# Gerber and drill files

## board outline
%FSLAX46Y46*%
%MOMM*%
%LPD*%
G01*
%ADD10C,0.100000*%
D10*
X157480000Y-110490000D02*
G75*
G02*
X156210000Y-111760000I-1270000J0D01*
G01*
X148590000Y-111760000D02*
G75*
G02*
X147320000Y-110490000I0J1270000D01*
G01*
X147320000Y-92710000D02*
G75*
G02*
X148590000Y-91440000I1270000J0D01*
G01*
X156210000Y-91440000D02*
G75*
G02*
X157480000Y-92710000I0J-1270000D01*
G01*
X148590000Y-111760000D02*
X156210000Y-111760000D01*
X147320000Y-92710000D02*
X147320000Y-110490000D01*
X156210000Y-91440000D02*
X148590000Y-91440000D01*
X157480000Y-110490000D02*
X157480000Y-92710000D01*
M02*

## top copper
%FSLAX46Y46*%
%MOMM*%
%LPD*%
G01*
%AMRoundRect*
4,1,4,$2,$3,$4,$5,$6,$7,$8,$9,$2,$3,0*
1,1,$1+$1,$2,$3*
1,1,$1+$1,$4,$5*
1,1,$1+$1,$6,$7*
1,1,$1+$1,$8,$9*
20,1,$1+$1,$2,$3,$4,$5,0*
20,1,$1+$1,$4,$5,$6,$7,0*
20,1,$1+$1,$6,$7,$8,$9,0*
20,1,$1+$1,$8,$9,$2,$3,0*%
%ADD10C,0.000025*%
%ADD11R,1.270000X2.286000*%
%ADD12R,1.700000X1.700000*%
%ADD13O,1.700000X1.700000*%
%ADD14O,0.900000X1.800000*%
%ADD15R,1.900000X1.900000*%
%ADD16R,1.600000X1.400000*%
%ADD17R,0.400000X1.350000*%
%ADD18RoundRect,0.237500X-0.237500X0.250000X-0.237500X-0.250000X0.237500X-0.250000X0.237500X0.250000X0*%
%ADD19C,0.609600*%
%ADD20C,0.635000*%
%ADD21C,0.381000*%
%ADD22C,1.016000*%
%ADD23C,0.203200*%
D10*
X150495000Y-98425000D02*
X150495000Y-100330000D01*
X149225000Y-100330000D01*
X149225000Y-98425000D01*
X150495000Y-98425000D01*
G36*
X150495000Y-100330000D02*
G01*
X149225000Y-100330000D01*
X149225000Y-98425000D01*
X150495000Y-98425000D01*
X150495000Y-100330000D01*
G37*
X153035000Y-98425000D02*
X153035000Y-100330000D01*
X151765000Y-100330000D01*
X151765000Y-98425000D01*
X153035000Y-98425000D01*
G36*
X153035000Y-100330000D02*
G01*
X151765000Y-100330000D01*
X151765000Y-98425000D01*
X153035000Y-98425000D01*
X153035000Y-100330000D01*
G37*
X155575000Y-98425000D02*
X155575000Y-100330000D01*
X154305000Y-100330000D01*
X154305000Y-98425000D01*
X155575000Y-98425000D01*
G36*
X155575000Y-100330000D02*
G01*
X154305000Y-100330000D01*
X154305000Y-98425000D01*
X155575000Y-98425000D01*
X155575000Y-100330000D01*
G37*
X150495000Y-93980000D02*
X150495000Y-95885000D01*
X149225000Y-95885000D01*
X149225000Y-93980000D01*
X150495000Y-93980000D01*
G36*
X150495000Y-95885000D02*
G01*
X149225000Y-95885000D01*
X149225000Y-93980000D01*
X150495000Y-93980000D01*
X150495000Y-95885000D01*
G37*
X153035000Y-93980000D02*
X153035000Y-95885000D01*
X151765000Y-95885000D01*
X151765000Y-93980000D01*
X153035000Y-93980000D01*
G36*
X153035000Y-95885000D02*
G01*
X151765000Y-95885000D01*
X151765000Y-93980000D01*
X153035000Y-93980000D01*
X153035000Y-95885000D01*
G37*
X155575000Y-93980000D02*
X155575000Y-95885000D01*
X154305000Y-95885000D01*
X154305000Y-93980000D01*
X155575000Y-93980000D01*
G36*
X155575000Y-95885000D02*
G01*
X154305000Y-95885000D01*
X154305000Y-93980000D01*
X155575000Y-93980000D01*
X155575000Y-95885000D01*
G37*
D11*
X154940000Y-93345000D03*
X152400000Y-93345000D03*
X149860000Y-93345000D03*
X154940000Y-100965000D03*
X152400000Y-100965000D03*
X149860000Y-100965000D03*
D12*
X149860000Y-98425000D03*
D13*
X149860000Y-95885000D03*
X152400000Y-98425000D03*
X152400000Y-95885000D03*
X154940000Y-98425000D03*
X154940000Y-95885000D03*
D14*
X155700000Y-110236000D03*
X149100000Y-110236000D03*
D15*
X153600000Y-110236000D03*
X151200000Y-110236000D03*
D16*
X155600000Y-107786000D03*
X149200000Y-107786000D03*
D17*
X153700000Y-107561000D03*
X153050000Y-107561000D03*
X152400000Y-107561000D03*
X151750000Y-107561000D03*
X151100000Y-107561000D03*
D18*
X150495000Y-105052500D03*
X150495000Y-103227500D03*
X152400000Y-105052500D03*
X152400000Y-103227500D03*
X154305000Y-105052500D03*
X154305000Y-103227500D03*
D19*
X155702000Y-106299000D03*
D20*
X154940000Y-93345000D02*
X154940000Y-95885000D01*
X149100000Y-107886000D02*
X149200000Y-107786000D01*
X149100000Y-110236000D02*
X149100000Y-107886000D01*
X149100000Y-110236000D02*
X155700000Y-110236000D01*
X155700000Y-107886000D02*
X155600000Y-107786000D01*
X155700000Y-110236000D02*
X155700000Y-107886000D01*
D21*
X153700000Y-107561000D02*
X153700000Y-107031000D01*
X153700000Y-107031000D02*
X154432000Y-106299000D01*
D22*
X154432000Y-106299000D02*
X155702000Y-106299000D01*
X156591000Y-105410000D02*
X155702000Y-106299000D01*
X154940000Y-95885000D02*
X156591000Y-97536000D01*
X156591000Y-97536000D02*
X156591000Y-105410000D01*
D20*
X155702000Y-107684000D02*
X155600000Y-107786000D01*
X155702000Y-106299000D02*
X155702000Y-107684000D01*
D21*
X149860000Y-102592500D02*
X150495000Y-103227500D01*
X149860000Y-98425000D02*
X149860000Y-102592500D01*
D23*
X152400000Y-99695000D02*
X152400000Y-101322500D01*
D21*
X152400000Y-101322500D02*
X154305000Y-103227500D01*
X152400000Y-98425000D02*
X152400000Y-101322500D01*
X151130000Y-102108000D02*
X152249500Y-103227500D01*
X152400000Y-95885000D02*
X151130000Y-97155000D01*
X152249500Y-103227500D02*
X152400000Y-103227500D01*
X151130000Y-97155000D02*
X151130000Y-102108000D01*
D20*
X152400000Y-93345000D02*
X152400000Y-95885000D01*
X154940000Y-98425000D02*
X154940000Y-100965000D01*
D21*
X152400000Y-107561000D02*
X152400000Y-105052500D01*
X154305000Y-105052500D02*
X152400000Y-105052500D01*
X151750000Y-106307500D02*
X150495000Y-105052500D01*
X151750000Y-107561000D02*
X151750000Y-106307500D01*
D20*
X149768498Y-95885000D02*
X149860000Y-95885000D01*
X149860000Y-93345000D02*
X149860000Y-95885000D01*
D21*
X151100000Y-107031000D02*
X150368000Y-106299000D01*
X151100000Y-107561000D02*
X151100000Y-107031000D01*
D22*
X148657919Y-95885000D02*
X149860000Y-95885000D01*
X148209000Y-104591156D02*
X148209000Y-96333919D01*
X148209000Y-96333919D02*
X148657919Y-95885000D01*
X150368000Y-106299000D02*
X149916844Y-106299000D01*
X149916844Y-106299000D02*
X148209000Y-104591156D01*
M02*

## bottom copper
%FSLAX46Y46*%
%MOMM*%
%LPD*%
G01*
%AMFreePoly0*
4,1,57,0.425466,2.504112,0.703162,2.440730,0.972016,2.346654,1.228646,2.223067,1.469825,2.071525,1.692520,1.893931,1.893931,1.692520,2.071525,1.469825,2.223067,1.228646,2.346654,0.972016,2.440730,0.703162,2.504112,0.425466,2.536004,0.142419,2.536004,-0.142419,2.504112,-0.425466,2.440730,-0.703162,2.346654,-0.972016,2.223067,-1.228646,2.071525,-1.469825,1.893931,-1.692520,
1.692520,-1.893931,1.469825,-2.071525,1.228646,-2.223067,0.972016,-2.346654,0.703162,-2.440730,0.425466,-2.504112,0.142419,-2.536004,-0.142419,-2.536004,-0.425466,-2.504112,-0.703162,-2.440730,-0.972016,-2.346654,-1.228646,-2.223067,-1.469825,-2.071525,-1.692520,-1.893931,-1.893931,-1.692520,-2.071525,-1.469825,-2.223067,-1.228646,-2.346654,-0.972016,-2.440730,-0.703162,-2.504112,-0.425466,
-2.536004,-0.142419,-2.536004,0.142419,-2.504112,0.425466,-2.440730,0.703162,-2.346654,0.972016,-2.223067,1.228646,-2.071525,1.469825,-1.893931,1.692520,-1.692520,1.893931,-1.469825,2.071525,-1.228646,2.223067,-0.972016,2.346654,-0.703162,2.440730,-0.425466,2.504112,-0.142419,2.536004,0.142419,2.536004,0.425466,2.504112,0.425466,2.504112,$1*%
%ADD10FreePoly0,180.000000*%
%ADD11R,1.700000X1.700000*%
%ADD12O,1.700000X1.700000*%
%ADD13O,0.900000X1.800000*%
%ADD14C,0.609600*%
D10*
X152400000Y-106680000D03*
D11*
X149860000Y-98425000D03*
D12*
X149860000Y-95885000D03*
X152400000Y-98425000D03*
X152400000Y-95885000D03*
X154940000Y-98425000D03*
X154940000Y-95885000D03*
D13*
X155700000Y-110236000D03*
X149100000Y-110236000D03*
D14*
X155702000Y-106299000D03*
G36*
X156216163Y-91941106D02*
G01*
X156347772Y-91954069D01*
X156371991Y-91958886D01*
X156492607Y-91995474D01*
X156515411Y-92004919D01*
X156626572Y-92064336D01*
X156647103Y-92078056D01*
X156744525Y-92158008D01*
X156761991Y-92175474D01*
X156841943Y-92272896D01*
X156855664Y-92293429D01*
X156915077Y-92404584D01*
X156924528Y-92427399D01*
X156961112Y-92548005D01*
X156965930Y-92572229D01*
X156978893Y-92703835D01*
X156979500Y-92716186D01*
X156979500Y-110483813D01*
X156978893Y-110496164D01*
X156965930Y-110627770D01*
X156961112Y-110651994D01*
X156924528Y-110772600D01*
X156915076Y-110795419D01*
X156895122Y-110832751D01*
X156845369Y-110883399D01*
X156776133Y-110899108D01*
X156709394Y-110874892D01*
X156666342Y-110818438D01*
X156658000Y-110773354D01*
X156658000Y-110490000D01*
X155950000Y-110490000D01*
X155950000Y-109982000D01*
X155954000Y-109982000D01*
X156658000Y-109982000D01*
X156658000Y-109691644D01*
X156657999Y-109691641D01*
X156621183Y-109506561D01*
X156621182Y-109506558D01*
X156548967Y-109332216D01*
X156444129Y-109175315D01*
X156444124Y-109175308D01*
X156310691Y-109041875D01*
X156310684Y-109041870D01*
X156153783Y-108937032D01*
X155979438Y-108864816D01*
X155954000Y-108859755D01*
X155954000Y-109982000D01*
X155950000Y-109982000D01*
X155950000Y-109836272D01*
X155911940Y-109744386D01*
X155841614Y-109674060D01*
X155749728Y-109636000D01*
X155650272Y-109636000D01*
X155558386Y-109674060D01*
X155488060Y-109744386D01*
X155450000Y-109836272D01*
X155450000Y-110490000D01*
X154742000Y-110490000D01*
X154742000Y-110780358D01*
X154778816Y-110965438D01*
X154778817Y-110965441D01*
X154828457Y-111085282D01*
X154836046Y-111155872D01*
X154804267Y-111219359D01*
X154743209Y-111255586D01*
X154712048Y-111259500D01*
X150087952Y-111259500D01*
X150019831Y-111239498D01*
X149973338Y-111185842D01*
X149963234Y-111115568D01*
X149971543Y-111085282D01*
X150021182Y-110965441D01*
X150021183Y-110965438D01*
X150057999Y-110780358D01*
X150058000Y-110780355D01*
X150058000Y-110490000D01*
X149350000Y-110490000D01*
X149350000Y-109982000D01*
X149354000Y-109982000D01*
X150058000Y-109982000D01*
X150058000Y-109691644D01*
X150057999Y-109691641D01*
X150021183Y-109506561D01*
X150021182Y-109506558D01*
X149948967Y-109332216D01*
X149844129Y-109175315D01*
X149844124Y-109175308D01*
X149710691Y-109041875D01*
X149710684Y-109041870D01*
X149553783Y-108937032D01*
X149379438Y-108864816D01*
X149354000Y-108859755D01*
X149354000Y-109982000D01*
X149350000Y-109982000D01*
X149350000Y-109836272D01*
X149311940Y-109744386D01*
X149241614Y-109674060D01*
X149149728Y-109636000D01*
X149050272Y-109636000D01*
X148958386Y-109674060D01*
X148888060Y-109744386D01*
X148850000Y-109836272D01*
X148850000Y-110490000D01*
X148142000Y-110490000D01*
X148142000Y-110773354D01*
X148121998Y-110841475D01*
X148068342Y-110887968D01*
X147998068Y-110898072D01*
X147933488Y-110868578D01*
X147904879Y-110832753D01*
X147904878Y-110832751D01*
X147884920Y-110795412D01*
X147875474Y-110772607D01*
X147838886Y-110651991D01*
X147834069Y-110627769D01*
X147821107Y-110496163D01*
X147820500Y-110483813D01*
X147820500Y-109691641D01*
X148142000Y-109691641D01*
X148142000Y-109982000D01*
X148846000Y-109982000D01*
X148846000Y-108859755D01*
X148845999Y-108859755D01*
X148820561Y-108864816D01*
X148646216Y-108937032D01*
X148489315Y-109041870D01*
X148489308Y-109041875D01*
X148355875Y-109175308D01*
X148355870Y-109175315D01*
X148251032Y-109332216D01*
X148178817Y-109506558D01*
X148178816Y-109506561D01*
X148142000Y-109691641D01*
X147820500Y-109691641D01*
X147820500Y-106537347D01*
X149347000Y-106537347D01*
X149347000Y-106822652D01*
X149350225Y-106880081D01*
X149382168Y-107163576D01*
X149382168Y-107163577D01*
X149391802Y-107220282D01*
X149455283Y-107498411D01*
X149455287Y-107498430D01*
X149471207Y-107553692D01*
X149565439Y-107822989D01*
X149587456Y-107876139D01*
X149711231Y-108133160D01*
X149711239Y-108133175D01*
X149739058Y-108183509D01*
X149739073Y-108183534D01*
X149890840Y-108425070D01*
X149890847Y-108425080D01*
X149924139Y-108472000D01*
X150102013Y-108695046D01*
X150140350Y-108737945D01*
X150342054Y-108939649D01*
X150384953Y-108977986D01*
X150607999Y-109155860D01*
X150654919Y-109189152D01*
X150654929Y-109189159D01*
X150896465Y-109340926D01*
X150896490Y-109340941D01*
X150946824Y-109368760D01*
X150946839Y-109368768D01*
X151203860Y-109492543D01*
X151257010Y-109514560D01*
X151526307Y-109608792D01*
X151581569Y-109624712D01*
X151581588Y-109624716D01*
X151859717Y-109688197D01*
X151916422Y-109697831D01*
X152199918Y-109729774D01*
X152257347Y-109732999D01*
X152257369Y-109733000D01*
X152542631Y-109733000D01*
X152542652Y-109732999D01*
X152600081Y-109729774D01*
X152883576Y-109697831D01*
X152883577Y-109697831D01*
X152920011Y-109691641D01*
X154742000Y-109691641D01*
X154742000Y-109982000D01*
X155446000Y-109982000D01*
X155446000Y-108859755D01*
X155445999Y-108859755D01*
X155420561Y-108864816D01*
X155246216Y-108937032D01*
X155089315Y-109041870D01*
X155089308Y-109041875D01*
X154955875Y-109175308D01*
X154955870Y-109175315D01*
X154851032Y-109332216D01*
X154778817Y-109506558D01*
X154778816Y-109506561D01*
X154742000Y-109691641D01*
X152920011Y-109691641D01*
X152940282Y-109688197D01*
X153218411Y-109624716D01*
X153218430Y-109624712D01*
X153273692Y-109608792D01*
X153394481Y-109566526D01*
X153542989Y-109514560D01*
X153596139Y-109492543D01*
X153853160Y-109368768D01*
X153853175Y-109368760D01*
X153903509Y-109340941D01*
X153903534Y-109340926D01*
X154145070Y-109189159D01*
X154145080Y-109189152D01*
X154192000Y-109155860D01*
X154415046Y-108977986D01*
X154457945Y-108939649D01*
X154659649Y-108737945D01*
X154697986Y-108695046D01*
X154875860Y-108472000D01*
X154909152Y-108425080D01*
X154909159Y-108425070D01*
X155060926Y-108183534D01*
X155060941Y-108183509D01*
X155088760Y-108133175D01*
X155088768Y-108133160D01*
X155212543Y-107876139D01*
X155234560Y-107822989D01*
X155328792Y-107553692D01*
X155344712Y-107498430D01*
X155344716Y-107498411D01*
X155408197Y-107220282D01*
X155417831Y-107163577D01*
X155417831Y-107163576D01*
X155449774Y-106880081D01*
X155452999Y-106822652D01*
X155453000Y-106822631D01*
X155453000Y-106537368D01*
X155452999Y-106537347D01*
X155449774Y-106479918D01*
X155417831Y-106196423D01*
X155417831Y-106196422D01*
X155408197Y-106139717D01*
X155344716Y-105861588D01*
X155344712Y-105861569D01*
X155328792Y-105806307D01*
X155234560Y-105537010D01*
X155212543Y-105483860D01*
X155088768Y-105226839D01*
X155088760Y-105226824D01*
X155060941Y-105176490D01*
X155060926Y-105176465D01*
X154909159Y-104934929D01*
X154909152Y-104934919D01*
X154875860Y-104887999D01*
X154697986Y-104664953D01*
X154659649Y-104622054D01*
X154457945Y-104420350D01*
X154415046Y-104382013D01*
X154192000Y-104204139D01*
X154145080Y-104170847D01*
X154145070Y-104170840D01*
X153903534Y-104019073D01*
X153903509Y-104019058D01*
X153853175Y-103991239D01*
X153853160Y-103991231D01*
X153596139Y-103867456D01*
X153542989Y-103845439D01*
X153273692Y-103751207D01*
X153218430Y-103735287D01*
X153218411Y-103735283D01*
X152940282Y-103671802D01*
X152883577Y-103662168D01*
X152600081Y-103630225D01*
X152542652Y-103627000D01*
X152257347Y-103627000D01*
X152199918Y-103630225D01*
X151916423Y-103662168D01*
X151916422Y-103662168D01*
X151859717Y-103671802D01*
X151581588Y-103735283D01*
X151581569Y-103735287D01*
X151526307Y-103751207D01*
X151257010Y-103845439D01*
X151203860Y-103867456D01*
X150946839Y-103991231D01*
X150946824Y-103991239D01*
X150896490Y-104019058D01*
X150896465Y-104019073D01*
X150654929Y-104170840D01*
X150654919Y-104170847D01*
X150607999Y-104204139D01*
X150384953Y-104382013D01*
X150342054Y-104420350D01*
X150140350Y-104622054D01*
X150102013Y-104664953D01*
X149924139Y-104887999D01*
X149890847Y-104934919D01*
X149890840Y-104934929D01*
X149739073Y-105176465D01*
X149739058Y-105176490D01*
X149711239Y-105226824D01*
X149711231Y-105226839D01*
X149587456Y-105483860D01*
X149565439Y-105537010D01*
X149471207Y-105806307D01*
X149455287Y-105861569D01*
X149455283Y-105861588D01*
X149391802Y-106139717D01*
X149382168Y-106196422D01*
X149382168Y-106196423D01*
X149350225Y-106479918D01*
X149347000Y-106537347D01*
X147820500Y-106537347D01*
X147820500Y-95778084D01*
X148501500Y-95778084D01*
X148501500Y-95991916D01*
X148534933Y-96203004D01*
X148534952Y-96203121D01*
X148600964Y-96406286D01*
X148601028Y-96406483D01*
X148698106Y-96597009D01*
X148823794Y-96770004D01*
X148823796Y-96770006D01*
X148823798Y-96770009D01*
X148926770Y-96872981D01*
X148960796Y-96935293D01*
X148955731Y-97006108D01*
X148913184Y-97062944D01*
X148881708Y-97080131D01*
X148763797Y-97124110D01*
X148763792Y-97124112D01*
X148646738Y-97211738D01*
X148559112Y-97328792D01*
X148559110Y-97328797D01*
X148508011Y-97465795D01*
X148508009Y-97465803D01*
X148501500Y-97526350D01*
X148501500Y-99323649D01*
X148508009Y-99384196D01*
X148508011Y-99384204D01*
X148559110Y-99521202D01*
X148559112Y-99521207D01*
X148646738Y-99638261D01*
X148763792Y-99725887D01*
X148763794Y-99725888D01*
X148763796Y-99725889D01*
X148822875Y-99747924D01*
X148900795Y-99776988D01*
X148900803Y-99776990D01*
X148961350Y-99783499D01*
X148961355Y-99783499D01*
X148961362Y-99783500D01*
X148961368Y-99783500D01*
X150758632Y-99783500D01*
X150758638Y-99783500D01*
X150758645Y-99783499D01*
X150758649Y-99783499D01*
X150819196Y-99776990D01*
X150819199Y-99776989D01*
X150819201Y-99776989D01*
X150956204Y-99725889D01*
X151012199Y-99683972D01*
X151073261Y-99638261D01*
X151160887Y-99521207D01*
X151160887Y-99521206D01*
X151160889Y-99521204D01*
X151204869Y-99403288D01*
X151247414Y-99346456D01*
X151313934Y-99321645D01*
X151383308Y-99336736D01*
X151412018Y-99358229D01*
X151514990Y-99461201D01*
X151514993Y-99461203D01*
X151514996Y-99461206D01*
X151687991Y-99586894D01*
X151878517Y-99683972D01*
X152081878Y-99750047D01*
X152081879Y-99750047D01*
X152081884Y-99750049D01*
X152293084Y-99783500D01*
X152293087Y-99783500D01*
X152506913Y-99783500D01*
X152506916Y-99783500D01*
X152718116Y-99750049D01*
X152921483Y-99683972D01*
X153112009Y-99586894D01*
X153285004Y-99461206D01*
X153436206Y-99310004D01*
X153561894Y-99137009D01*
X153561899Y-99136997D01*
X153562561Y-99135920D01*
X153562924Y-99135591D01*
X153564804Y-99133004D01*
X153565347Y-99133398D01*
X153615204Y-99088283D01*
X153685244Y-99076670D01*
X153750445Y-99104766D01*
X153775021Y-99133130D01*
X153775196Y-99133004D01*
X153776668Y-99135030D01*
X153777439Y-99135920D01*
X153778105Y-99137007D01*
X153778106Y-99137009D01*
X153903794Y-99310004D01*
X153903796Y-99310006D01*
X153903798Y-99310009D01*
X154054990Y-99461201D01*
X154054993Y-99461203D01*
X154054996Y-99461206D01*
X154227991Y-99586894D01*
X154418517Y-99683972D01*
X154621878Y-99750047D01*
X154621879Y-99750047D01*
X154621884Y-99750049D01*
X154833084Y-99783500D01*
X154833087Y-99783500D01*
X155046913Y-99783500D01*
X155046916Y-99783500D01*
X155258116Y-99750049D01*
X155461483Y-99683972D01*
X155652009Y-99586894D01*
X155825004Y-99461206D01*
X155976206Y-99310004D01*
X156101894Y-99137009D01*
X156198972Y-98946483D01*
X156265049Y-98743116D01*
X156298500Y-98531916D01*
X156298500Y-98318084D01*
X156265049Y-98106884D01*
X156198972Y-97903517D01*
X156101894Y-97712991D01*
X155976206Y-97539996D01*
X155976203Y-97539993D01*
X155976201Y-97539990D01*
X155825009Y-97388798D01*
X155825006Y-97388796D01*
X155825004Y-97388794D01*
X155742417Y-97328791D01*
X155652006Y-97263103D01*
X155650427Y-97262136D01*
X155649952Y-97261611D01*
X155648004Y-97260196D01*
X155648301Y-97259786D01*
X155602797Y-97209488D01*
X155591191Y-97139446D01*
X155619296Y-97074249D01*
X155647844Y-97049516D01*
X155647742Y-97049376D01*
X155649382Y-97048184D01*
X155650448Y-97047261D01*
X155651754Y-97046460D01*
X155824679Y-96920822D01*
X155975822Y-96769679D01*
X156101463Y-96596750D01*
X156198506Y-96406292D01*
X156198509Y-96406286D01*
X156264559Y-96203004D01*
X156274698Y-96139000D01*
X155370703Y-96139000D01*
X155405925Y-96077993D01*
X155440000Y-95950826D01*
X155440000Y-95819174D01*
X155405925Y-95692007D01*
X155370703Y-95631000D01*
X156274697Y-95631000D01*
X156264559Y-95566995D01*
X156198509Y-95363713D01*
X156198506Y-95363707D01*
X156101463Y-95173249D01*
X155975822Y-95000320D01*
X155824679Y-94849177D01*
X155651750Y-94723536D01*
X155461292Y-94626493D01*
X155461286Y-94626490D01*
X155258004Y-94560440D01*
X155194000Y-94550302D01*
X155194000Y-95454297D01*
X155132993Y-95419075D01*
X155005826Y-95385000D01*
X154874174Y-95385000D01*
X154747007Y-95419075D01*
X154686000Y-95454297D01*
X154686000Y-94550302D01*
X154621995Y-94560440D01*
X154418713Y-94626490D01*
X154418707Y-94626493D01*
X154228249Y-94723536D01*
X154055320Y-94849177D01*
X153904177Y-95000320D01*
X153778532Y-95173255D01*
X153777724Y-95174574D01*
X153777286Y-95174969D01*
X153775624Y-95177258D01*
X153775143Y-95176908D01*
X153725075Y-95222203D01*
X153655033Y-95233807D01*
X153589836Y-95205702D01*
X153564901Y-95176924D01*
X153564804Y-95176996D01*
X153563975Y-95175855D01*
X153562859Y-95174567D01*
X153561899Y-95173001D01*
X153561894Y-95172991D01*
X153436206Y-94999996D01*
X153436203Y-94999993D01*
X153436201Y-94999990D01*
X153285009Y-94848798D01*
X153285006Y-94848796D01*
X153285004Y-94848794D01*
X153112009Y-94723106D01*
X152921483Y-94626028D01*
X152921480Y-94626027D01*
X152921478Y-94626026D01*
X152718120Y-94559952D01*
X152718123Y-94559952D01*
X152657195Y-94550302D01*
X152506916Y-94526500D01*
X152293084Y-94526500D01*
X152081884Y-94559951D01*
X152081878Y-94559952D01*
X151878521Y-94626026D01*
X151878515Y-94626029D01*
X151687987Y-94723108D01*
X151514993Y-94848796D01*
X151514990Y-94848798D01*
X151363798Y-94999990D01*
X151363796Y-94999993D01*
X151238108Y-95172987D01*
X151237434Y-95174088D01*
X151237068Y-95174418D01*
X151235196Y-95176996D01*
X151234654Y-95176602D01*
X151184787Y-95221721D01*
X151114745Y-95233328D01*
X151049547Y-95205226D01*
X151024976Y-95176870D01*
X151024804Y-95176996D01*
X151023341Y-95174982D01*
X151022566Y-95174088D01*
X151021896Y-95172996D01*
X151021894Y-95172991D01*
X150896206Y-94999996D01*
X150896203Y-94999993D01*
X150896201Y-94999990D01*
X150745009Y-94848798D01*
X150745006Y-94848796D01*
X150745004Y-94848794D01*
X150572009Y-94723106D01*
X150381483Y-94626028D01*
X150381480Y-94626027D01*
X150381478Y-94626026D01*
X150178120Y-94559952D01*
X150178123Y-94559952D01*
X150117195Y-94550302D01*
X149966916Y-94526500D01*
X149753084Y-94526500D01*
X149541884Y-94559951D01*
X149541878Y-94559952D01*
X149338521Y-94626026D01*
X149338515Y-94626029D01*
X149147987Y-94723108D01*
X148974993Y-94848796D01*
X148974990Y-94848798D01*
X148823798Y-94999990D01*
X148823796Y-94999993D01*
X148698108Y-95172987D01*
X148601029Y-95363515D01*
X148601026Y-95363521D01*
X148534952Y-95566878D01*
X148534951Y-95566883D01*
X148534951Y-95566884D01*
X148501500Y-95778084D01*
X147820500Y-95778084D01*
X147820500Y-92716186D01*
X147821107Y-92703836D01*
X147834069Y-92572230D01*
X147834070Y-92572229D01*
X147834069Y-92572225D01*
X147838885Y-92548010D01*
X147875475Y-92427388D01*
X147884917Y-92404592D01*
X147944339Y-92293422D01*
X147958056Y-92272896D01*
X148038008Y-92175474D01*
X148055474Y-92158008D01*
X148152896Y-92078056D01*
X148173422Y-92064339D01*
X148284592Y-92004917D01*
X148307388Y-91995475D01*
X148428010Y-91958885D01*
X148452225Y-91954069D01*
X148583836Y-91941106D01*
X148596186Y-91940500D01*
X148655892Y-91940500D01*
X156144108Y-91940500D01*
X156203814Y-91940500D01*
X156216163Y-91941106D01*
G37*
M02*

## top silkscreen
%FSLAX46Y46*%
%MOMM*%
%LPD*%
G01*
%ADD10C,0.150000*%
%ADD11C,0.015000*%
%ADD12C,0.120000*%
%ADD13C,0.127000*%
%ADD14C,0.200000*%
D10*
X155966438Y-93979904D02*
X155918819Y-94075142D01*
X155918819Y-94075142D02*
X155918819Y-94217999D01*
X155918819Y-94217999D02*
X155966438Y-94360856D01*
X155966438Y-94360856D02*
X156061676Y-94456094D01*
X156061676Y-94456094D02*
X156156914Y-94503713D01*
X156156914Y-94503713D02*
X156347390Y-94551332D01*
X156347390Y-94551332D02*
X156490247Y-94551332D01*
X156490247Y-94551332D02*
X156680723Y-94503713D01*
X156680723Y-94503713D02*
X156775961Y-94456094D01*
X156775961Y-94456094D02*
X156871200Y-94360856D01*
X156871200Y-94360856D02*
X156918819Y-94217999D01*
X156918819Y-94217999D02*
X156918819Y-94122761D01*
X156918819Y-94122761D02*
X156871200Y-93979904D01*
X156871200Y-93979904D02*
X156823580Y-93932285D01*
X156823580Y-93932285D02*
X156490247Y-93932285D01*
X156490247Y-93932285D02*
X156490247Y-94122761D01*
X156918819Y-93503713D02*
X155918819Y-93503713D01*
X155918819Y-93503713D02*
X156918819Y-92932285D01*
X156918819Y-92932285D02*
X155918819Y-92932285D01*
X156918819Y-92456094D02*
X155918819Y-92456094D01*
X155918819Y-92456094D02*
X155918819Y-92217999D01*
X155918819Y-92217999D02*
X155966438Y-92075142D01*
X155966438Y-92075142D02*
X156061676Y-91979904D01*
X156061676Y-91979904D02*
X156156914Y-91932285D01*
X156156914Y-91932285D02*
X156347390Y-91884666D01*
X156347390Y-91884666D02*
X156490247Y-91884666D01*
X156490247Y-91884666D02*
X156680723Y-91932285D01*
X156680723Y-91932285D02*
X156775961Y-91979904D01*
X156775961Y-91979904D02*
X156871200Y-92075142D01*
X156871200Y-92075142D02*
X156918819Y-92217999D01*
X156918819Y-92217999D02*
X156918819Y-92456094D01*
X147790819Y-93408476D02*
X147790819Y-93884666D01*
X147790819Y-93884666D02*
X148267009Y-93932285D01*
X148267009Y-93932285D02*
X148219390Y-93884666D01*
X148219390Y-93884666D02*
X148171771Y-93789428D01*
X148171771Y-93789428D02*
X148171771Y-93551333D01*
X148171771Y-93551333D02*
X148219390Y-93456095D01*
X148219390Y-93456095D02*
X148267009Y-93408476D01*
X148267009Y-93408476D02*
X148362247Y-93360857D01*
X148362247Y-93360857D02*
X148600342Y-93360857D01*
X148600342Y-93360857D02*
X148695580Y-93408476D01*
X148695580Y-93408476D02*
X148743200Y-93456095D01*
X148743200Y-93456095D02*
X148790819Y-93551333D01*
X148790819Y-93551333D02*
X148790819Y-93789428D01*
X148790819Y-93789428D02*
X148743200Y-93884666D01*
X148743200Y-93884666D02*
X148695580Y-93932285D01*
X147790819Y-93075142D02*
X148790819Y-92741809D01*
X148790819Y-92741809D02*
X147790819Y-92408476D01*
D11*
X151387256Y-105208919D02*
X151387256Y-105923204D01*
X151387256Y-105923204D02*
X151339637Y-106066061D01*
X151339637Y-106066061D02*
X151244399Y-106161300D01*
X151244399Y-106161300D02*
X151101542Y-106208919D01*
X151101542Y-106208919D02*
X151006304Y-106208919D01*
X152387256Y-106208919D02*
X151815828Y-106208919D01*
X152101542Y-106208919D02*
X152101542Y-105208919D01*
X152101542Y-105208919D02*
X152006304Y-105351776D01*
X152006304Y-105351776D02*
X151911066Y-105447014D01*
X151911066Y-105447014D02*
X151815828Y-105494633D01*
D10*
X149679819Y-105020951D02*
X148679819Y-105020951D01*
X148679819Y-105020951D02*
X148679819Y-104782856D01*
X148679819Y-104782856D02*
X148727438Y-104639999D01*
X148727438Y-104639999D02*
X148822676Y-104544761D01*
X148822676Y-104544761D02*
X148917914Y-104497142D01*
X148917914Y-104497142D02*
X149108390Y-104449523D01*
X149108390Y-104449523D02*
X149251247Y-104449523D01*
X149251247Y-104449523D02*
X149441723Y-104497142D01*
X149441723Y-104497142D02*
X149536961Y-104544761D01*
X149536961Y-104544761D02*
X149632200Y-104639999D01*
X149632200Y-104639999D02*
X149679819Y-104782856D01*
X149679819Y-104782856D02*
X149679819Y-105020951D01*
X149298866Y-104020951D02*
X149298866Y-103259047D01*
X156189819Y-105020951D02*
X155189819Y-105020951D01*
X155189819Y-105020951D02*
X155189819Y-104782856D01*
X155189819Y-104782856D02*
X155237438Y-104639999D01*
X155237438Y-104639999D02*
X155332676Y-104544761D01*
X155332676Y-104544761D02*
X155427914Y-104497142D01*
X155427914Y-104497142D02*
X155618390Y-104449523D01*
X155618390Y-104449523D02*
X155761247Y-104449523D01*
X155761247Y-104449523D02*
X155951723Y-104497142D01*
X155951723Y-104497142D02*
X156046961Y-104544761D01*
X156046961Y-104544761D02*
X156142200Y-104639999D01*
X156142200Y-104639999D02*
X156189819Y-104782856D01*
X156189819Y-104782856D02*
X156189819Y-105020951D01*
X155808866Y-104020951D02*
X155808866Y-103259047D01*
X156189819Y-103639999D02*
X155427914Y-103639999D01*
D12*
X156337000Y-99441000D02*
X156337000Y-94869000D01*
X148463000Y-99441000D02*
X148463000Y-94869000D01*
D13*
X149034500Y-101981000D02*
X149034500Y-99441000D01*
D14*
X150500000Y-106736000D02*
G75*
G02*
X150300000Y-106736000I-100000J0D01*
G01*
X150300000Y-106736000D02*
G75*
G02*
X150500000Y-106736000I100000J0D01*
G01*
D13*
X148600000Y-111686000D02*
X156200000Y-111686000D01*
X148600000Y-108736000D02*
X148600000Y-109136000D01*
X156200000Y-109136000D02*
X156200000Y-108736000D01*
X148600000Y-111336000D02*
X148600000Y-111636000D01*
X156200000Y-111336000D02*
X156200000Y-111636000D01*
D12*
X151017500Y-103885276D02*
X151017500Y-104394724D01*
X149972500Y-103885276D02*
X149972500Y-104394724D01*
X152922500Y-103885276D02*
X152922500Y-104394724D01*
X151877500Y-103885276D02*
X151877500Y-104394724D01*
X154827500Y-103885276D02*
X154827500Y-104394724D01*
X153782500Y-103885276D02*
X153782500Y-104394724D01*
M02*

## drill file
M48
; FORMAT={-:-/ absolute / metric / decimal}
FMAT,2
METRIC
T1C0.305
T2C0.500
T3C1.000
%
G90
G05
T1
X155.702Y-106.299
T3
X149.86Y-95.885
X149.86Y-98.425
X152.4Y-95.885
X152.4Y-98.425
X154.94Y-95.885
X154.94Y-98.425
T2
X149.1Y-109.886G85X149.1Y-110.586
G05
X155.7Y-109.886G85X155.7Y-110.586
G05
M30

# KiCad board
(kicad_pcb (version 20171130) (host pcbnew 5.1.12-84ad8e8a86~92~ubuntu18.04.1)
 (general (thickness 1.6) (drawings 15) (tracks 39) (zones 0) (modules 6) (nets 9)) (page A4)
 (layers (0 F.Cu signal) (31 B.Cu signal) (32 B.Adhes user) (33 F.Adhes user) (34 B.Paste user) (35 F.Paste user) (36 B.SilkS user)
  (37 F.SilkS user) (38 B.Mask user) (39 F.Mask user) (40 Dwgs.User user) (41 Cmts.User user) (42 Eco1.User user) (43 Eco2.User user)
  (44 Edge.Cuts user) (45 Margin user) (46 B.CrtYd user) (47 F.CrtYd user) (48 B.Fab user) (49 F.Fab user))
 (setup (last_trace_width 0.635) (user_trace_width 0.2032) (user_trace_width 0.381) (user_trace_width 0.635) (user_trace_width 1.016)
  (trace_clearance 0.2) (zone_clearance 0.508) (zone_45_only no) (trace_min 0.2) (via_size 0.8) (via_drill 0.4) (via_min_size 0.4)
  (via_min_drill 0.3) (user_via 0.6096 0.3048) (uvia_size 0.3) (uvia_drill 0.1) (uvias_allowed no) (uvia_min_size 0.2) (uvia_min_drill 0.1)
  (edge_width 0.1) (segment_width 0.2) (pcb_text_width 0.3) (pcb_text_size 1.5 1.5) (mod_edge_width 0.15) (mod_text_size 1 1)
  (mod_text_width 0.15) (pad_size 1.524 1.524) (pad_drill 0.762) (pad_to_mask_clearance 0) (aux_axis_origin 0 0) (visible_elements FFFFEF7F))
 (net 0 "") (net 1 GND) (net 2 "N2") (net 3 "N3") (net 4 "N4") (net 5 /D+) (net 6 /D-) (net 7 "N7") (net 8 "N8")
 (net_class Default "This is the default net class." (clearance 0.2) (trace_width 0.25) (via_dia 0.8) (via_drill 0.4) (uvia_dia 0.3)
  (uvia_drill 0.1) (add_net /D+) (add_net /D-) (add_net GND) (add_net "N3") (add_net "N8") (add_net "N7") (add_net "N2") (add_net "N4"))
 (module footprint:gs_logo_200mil (layer B.Cu) (at 152.4 106.68 180)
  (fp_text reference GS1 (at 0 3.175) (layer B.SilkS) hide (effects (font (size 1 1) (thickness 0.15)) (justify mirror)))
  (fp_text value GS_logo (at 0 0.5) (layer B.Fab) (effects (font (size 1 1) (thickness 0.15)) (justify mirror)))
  (pad 1 smd custom (at 0 0 180) (size 5.08 5.08) (layers B.Cu) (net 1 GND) (zone_connect 0) (options (clearance outline) (anchor circle))
   (primitives)))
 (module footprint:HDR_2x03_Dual (layer F.Cu) (at 149.86 98.425 90)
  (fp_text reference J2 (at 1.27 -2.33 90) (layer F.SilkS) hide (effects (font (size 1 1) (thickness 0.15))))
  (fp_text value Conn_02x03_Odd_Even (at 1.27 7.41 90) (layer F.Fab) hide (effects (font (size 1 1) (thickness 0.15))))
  (fp_line (start -1.016 6.477) (end 3.556 6.477) (layer F.SilkS) (width 0.12))
  (fp_line (start -1.016 -1.397) (end 3.556 -1.397) (layer F.SilkS) (width 0.12))
  (fp_line (start -3.556 -0.8255) (end -1.016 -0.8255) (layer F.SilkS) (width 0.127))
  (fp_poly (pts (xy 0 0.635) (xy -1.905 0.635) (xy -1.905 -0.635) (xy 0 -0.635)) (layer F.Cu) (width 0.000025))
  (fp_poly (pts (xy 0 3.175) (xy -1.905 3.175) (xy -1.905 1.905) (xy 0 1.905)) (layer F.Cu) (width 0.000025))
  (fp_poly (pts (xy 0 5.715) (xy -1.905 5.715) (xy -1.905 4.445) (xy 0 4.445)) (layer F.Cu) (width 0.000025))
  (fp_poly (pts (xy 4.445 0.635) (xy 2.54 0.635) (xy 2.54 -0.635) (xy 4.445 -0.635)) (layer F.Cu) (width 0.000025))
  (fp_poly (pts (xy 4.445 3.175) (xy 2.54 3.175) (xy 2.54 1.905) (xy 4.445 1.905)) (layer F.Cu) (width 0.000025))
  (fp_poly (pts (xy 4.445 5.715) (xy 2.54 5.715) (xy 2.54 4.445) (xy 4.445 4.445)) (layer F.Cu) (width 0.000025))
  (pad 6 smd rect (at 5.08 5.08 90) (size 2.286 1.27) (layers F.Cu F.Paste F.Mask) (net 1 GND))
  (pad 4 smd rect (at 5.08 2.54 90) (size 2.286 1.27) (layers F.Cu F.Paste F.Mask) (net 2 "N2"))
  (pad 2 smd rect (at 5.08 0 90) (size 2.286 1.27) (layers F.Cu F.Paste F.Mask) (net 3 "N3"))
  (pad 5 smd rect (at -2.54 5.08 90) (size 2.286 1.27) (layers F.Cu F.Paste F.Mask) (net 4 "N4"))
  (pad 3 smd rect (at -2.54 2.54 90) (size 2.286 1.27) (layers F.Cu F.Paste F.Mask) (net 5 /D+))
  (pad 1 smd rect (at -2.54 0 90) (size 2.286 1.27) (layers F.Cu F.Paste F.Mask) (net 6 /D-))
  (pad 1 thru_hole rect (at 0 0 90) (size 1.7 1.7) (drill 1) (layers *.Cu *.Mask) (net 6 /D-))
  (pad 2 thru_hole oval (at 2.54 0 90) (size 1.7 1.7) (drill 1) (layers *.Cu *.Mask) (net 3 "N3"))
  (pad 3 thru_hole oval (at 0 2.54 90) (size 1.7 1.7) (drill 1) (layers *.Cu *.Mask) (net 5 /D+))
  (pad 4 thru_hole oval (at 2.54 2.54 90) (size 1.7 1.7) (drill 1) (layers *.Cu *.Mask) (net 2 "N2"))
  (pad 5 thru_hole oval (at 0 5.08 90) (size 1.7 1.7) (drill 1) (layers *.Cu *.Mask) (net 4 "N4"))
  (pad 6 thru_hole oval (at 2.54 5.08 90) (size 1.7 1.7) (drill 1) (layers *.Cu *.Mask) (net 1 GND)))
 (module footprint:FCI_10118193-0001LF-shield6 (layer F.Cu) (at 152.4 110.236)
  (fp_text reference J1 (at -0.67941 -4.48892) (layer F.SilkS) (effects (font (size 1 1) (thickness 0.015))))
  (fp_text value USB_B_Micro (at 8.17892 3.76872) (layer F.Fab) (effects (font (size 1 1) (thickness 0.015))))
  (fp_circle (center -2 -3.5) (end -1.9 -3.5) (layer F.SilkS) (width 0.2))
  (fp_line (start -3.8 1.45) (end 3.8 1.45) (layer F.SilkS) (width 0.127))
  (fp_line (start -3.8 -1.5) (end -3.8 -1.1) (layer F.SilkS) (width 0.127))
  (fp_line (start 3.8 -1.1) (end 3.8 -1.5) (layer F.SilkS) (width 0.127))
  (fp_line (start -3.8 1.1) (end -3.8 1.4) (layer F.SilkS) (width 0.127))
  (fp_line (start 3.8 1.1) (end 3.8 1.4) (layer F.SilkS) (width 0.127))
  (pad 6 thru_hole oval (at 3.3 0) (size 0.9 1.8) (drill oval 0.5 1.2) (layers *.Cu *.Mask) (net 1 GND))
  (pad 6 thru_hole oval (at -3.3 0) (size 0.9 1.8) (drill oval 0.5 1.2) (layers *.Cu *.Mask) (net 1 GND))
  (pad 6 smd rect (at 1.2 0) (size 1.9 1.9) (layers F.Cu F.Paste F.Mask) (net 1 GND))
  (pad 6 smd rect (at -1.2 0) (size 1.9 1.9) (layers F.Cu F.Paste F.Mask) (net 1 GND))
  (pad 6 smd rect (at 3.2 -2.45) (size 1.6 1.4) (layers F.Cu F.Paste F.Mask) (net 1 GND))
  (pad 6 smd rect (at -3.2 -2.45) (size 1.6 1.4) (layers F.Cu F.Paste F.Mask) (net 1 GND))
  (pad 5 smd rect (at 1.3 -2.675) (size 0.4 1.35) (layers F.Cu F.Paste F.Mask) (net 1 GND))
  (pad 4 smd rect (at 0.65 -2.675) (size 0.4 1.35) (layers F.Cu F.Paste F.Mask))
  (pad 3 smd rect (at 0 -2.675) (size 0.4 1.35) (layers F.Cu F.Paste F.Mask) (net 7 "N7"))
  (pad 2 smd rect (at -0.65 -2.675) (size 0.4 1.35) (layers F.Cu F.Paste F.Mask) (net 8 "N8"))
  (pad 1 smd rect (at -1.3 -2.675) (size 0.4 1.35) (layers F.Cu F.Paste F.Mask) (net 3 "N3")))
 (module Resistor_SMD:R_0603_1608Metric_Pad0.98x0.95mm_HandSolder (layer F.Cu) (at 150.495 104.14 270)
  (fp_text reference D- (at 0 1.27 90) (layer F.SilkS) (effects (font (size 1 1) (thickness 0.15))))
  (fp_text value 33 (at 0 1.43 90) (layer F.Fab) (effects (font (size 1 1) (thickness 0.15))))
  (fp_line (start -0.254724 -0.5225) (end 0.254724 -0.5225) (layer F.SilkS) (width 0.12))
  (fp_line (start -0.254724 0.5225) (end 0.254724 0.5225) (layer F.SilkS) (width 0.12))
  (pad 2 smd roundrect (at 0.9125 0 270) (size 0.975 0.95) (layers F.Cu F.Paste F.Mask) (roundrect_rratio 0.25) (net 8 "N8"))
  (pad 1 smd roundrect (at -0.9125 0 270) (size 0.975 0.95) (layers F.Cu F.Paste F.Mask) (roundrect_rratio 0.25) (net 6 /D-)))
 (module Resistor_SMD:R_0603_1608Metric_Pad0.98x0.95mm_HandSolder (layer F.Cu) (at 152.4 104.14 270)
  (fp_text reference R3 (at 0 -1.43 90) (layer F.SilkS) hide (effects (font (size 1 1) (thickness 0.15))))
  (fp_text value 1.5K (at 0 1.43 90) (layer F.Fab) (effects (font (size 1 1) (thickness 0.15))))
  (fp_line (start -0.254724 -0.5225) (end 0.254724 -0.5225) (layer F.SilkS) (width 0.12))
  (fp_line (start -0.254724 0.5225) (end 0.254724 0.5225) (layer F.SilkS) (width 0.12))
  (pad 2 smd roundrect (at 0.9125 0 270) (size 0.975 0.95) (layers F.Cu F.Paste F.Mask) (roundrect_rratio 0.25) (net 7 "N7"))
  (pad 1 smd roundrect (at -0.9125 0 270) (size 0.975 0.95) (layers F.Cu F.Paste F.Mask) (roundrect_rratio 0.25) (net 2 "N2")))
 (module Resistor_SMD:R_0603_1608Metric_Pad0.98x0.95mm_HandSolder (layer F.Cu) (at 154.305 104.14 270)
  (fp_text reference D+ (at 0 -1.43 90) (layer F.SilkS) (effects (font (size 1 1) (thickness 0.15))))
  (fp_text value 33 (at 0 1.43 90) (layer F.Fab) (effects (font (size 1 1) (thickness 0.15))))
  (fp_line (start -0.254724 -0.5225) (end 0.254724 -0.5225) (layer F.SilkS) (width 0.12))
  (fp_line (start -0.254724 0.5225) (end 0.254724 0.5225) (layer F.SilkS) (width 0.12))
  (pad 2 smd roundrect (at 0.9125 0 270) (size 0.975 0.95) (layers F.Cu F.Paste F.Mask) (roundrect_rratio 0.25) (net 7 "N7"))
  (pad 1 smd roundrect (at -0.9125 0 270) (size 0.975 0.95) (layers F.Cu F.Paste F.Mask) (roundrect_rratio 0.25) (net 5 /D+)))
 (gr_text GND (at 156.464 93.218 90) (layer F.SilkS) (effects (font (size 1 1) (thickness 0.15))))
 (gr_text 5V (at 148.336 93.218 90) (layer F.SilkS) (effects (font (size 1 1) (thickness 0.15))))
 (gr_arc (start 156.21 110.49) (end 156.21 111.76) (angle -90) (layer Edge.Cuts) (width 0.1))
 (gr_arc (start 148.59 110.49) (end 147.32 110.49) (angle -90) (layer Edge.Cuts) (width 0.1))
 (gr_arc (start 148.59 92.71) (end 148.59 91.44) (angle -90) (layer Edge.Cuts) (width 0.1))
 (gr_arc (start 156.21 92.71) (end 157.48 92.71) (angle -90) (layer Edge.Cuts) (width 0.1))
 (gr_line (start 148.59 111.76) (end 156.21 111.76) (layer Edge.Cuts) (width 0.1))
 (gr_line (start 147.32 92.71) (end 147.32 110.49) (layer Edge.Cuts) (width 0.1))
 (gr_line (start 156.21 91.44) (end 148.59 91.44) (layer Edge.Cuts) (width 0.1))
 (gr_line (start 157.48 110.49) (end 157.48 92.71) (layer Edge.Cuts) (width 0.1))
 (segment (start 154.94 93.345) (end 154.94 95.885) (width 0.635) (layer F.Cu) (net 1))
 (segment (start 149.1 107.886) (end 149.2 107.786) (width 0.635) (layer F.Cu) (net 1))
 (segment (start 149.1 110.236) (end 149.1 107.886) (width 0.635) (layer F.Cu) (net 1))
 (segment (start 149.1 110.236) (end 155.7 110.236) (width 0.635) (layer F.Cu) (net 1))
 (segment (start 155.7 107.886) (end 155.6 107.786) (width 0.635) (layer F.Cu) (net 1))
 (segment (start 155.7 110.236) (end 155.7 107.886) (width 0.635) (layer F.Cu) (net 1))
 (via (at 155.702 106.299) (size 0.6096) (drill 0.3048) (layers F.Cu B.Cu) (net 1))
 (segment (start 153.7 107.561) (end 153.7 107.031) (width 0.381) (layer F.Cu) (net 1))
 (segment (start 153.7 107.031) (end 154.432 106.299) (width 0.381) (layer F.Cu) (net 1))
 (segment (start 154.432 106.299) (end 155.702 106.299) (width 1.016) (layer F.Cu) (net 1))
 (segment (start 156.591 105.41) (end 155.702 106.299) (width 1.016) (layer F.Cu) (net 1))
 (segment (start 154.94 95.885) (end 156.591 97.536) (width 1.016) (layer F.Cu) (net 1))
 (segment (start 156.591 97.536) (end 156.591 105.41) (width 1.016) (layer F.Cu) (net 1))
 (segment (start 155.702 107.684) (end 155.6 107.786) (width 0.635) (layer F.Cu) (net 1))
 (segment (start 155.702 106.299) (end 155.702 107.684) (width 0.635) (layer F.Cu) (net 1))
 (segment (start 149.86 102.5925) (end 150.495 103.2275) (width 0.381) (layer F.Cu) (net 6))
 (segment (start 149.86 98.425) (end 149.86 102.5925) (width 0.381) (layer F.Cu) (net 6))
 (segment (start 152.4 99.695) (end 152.4 101.3225) (width 0.2032) (layer F.Cu) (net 5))
 (segment (start 152.4 101.3225) (end 154.305 103.2275) (width 0.381) (layer F.Cu) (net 5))
 (segment (start 152.4 98.425) (end 152.4 101.3225) (width 0.381) (layer F.Cu) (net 5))
 (segment (start 151.13 102.108) (end 152.2495 103.2275) (width 0.381) (layer F.Cu) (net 2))
 (segment (start 152.4 95.885) (end 151.13 97.155) (width 0.381) (layer F.Cu) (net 2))
 (segment (start 152.2495 103.2275) (end 152.4 103.2275) (width 0.381) (layer F.Cu) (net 2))
 (segment (start 151.13 97.155) (end 151.13 102.108) (width 0.381) (layer F.Cu) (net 2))
 (segment (start 152.4 93.345) (end 152.4 95.885) (width 0.635) (layer F.Cu) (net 2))
 (segment (start 154.94 98.425) (end 154.94 100.965) (width 0.635) (layer F.Cu) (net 4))
 (segment (start 152.4 107.561) (end 152.4 105.0525) (width 0.381) (layer F.Cu) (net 7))
 (segment (start 154.305 105.0525) (end 152.4 105.0525) (width 0.381) (layer F.Cu) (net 7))
 (segment (start 151.75 106.3075) (end 150.495 105.0525) (width 0.381) (layer F.Cu) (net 8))
 (segment (start 151.75 107.561) (end 151.75 106.3075) (width 0.381) (layer F.Cu) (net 8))
 (segment (start 149.768498 95.885) (end 149.86 95.885) (width 0.635) (layer F.Cu) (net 3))
 (segment (start 149.86 93.345) (end 149.86 95.885) (width 0.635) (layer F.Cu) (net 3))
 (segment (start 151.1 107.031) (end 150.368 106.299) (width 0.381) (layer F.Cu) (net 3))
 (segment (start 151.1 107.561) (end 151.1 107.031) (width 0.381) (layer F.Cu) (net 3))
 (segment (start 148.657919 95.885) (end 149.86 95.885) (width 1.016) (layer F.Cu) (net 3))
 (segment (start 148.209 104.591156) (end 148.209 96.333919) (width 1.016) (layer F.Cu) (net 3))
 (segment (start 148.209 96.333919) (end 148.657919 95.885) (width 1.016) (layer F.Cu) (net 3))
 (segment (start 150.368 106.299) (end 149.916844 106.299) (width 1.016) (layer F.Cu) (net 3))
 (segment (start 149.916844 106.299) (end 148.209 104.591156) (width 1.016) (layer F.Cu) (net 3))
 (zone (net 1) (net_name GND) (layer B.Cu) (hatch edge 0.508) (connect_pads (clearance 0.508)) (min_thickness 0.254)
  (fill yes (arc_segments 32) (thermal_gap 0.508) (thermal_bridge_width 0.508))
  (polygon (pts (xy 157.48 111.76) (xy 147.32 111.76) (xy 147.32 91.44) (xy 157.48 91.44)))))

